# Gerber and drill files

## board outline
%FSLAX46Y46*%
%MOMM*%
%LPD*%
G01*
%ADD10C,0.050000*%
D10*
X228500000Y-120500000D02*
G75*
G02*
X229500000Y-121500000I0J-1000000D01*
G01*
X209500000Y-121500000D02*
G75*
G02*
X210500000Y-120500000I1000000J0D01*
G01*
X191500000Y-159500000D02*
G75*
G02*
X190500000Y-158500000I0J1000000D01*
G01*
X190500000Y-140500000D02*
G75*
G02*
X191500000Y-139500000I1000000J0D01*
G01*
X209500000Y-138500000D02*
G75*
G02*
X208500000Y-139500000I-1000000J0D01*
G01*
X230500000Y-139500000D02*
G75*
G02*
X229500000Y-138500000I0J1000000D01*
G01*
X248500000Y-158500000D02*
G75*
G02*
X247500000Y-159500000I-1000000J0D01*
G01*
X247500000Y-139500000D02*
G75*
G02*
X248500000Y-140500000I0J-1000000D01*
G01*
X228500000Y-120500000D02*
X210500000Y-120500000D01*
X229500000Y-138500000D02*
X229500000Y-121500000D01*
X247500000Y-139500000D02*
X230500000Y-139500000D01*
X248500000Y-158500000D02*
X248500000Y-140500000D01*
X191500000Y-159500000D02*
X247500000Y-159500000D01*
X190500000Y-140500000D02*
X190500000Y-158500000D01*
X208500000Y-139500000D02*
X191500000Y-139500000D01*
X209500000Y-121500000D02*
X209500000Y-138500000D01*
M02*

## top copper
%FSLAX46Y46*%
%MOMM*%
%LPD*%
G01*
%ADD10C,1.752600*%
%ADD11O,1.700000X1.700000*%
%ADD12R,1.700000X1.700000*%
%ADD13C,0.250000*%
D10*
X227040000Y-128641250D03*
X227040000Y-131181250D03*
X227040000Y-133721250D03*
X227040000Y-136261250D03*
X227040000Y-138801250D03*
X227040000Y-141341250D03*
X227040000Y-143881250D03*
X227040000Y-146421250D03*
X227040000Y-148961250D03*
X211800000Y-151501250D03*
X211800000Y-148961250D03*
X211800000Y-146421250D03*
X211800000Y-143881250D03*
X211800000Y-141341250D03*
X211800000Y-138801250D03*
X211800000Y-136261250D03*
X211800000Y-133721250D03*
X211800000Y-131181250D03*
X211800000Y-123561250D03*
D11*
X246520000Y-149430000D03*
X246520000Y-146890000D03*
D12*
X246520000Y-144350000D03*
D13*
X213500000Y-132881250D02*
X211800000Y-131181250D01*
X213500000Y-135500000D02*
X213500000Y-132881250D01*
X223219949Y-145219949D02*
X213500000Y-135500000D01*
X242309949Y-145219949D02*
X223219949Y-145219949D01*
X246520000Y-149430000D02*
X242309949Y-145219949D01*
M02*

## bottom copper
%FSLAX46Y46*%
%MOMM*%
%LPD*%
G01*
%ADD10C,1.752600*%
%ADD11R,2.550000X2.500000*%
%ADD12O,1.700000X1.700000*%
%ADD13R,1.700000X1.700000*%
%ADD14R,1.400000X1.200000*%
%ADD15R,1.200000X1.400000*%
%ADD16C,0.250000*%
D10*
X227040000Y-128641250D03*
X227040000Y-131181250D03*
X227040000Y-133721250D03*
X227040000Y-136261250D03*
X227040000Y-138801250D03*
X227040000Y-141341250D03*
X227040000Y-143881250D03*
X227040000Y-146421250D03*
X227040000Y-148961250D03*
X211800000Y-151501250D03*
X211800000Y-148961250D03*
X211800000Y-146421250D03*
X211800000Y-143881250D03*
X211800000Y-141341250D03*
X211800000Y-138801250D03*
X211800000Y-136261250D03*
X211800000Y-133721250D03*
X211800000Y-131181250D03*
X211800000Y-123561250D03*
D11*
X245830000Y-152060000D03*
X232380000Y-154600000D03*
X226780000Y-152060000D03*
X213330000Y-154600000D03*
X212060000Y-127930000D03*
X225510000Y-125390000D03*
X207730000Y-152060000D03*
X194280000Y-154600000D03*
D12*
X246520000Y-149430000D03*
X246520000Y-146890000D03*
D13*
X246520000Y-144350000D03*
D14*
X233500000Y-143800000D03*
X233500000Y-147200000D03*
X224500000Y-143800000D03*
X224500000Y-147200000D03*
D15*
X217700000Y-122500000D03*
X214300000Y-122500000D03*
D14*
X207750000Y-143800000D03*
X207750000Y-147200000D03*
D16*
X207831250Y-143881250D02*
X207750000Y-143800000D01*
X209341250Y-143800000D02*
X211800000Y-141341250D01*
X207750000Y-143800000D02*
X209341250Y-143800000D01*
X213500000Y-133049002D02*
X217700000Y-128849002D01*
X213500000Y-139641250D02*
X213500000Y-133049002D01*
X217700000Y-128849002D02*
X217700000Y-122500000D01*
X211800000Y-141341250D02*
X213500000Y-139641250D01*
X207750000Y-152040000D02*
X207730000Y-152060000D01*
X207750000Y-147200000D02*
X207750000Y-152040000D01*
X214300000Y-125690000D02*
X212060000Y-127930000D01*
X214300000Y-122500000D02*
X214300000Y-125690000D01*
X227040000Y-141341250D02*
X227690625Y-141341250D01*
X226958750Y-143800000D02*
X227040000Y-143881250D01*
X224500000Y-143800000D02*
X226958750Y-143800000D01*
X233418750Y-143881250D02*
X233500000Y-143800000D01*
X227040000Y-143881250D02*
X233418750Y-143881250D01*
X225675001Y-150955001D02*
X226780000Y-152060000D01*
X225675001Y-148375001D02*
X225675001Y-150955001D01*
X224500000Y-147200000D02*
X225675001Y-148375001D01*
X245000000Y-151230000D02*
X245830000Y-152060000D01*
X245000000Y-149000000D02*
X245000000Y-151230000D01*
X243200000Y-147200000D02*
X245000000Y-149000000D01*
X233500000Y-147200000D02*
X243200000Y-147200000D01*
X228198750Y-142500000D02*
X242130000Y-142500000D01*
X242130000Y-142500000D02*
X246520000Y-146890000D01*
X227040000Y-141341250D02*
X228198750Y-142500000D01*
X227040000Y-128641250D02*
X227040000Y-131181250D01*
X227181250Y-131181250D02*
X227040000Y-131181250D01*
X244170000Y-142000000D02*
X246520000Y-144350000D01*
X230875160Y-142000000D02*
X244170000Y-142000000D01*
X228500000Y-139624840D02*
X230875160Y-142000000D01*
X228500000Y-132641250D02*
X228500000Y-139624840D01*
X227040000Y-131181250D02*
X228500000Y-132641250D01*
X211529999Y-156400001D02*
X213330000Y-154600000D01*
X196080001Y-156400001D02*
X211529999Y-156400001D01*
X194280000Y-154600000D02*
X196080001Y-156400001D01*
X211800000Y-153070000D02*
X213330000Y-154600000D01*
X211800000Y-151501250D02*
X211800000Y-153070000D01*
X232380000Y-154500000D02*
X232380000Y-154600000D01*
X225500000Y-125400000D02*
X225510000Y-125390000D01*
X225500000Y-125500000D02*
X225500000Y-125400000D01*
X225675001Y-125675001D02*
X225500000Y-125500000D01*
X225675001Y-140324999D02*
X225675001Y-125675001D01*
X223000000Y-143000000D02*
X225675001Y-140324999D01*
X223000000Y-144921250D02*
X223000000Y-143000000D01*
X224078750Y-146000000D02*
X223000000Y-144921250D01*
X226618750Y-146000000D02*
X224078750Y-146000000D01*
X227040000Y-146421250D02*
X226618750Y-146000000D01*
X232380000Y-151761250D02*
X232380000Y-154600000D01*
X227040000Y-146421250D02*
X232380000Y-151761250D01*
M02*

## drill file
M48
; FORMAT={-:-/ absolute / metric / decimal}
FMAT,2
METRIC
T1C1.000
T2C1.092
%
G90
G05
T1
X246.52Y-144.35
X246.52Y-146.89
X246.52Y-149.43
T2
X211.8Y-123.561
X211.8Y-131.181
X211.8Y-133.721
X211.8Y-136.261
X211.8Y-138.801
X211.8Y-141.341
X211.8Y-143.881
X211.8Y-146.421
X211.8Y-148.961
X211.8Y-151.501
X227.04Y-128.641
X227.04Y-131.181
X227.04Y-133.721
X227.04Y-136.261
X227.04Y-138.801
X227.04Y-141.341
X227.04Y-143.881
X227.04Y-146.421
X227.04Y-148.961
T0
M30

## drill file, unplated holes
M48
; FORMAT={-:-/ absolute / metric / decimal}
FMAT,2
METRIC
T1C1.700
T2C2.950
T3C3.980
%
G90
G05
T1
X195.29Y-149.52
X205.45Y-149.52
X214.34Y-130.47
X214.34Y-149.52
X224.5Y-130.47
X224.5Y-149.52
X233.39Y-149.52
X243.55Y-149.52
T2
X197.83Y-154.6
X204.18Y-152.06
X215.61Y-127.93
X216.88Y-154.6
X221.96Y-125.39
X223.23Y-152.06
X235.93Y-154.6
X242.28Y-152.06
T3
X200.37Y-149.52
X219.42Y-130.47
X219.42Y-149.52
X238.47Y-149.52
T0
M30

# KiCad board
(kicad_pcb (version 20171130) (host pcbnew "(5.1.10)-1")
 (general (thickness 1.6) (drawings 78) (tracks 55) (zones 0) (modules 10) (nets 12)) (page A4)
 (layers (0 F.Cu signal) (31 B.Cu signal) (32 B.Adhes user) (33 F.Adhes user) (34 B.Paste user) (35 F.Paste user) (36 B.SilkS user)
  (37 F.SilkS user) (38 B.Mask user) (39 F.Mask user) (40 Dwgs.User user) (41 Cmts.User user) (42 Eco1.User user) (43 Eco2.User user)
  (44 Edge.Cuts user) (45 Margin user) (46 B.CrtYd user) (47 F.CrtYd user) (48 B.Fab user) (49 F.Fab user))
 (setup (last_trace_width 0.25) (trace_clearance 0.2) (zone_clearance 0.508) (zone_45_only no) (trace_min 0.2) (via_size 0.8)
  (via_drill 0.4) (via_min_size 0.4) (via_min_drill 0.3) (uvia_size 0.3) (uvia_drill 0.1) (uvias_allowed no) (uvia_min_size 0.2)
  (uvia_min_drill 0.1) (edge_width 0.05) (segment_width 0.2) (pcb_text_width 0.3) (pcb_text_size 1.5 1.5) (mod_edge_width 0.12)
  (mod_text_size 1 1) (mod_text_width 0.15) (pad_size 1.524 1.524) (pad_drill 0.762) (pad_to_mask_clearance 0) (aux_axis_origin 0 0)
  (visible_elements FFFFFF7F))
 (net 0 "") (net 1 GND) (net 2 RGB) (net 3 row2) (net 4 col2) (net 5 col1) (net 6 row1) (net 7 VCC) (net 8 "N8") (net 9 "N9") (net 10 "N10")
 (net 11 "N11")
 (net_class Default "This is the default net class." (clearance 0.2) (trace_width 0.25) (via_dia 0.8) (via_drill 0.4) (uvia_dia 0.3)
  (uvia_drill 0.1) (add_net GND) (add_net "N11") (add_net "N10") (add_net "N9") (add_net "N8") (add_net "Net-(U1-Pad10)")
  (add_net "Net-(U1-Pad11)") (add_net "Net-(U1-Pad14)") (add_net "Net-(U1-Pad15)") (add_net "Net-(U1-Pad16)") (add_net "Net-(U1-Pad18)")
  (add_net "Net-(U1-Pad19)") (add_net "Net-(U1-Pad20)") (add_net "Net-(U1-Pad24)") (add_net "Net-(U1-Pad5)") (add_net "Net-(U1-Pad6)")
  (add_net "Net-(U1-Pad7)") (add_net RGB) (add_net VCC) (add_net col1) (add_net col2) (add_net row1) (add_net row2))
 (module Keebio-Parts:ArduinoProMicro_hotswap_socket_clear (layer B.Cu) (at 219.42 137.53125 270)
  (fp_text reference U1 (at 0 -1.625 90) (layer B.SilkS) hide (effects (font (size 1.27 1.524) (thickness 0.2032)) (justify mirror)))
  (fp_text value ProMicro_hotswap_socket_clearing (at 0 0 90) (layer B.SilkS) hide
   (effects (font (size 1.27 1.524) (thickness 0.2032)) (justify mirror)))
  (pad 3 thru_hole circle (at -8.89 -7.62 270) (size 1.7526 1.7526) (drill 1.0922) (layers *.Cu *.SilkS *.Mask) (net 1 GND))
  (pad 4 thru_hole circle (at -6.35 -7.62 270) (size 1.7526 1.7526) (drill 1.0922) (layers *.Cu *.SilkS *.Mask) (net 1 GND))
  (pad 5 thru_hole circle (at -3.81 -7.62 270) (size 1.7526 1.7526) (drill 1.0922) (layers *.Cu *.SilkS *.Mask))
  (pad 6 thru_hole circle (at -1.27 -7.62 270) (size 1.7526 1.7526) (drill 1.0922) (layers *.Cu *.SilkS *.Mask))
  (pad 7 thru_hole circle (at 1.27 -7.62 270) (size 1.7526 1.7526) (drill 1.0922) (layers *.Cu *.SilkS *.Mask))
  (pad 8 thru_hole circle (at 3.81 -7.62 270) (size 1.7526 1.7526) (drill 1.0922) (layers *.Cu *.SilkS *.Mask) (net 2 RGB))
  (pad 9 thru_hole circle (at 6.35 -7.62 270) (size 1.7526 1.7526) (drill 1.0922) (layers *.Cu *.SilkS *.Mask) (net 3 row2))
  (pad 10 thru_hole circle (at 8.89 -7.62 270) (size 1.7526 1.7526) (drill 1.0922) (layers *.Cu *.SilkS *.Mask) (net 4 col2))
  (pad 11 thru_hole circle (at 11.43 -7.62 270) (size 1.7526 1.7526) (drill 1.0922) (layers *.Cu *.SilkS *.Mask))
  (pad 13 thru_hole circle (at 13.97 7.62 270) (size 1.7526 1.7526) (drill 1.0922) (layers *.Cu *.SilkS *.Mask) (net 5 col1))
  (pad 14 thru_hole circle (at 11.43 7.62 270) (size 1.7526 1.7526) (drill 1.0922) (layers *.Cu *.SilkS *.Mask))
  (pad 15 thru_hole circle (at 8.89 7.62 270) (size 1.7526 1.7526) (drill 1.0922) (layers *.Cu *.SilkS *.Mask))
  (pad 16 thru_hole circle (at 6.35 7.62 270) (size 1.7526 1.7526) (drill 1.0922) (layers *.Cu *.SilkS *.Mask))
  (pad 17 thru_hole circle (at 3.81 7.62 270) (size 1.7526 1.7526) (drill 1.0922) (layers *.Cu *.SilkS *.Mask) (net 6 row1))
  (pad 18 thru_hole circle (at 1.27 7.62 270) (size 1.7526 1.7526) (drill 1.0922) (layers *.Cu *.SilkS *.Mask))
  (pad 19 thru_hole circle (at -1.27 7.62 270) (size 1.7526 1.7526) (drill 1.0922) (layers *.Cu *.SilkS *.Mask))
  (pad 20 thru_hole circle (at -3.81 7.62 270) (size 1.7526 1.7526) (drill 1.0922) (layers *.Cu *.SilkS *.Mask))
  (pad 21 thru_hole circle (at -6.35 7.62 270) (size 1.7526 1.7526) (drill 1.0922) (layers *.Cu *.SilkS *.Mask) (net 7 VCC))
  (pad 24 thru_hole circle (at -13.97 7.62 270) (size 1.7526 1.7526) (drill 1.0922) (layers *.Cu *.SilkS *.Mask)))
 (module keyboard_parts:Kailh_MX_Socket (layer F.Cu) (at 238.47 149.52)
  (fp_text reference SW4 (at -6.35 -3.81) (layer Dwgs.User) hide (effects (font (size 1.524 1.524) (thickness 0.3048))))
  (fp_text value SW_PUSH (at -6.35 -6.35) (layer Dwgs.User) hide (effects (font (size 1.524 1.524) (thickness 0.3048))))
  (pad 1 smd rect (at 7.36 2.54) (size 2.55 2.5) (layers B.Cu B.Paste B.Mask) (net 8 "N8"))
  (pad "" np_thru_hole circle (at 0 0) (size 3.98018 3.98018) (drill 3.98018) (layers *.Cu *.Mask))
  (pad "" np_thru_hole circle (at -2.54 5.08) (size 2.95 2.95) (drill 2.95) (layers *.Cu *.Mask))
  (pad "" np_thru_hole circle (at 3.81 2.54) (size 2.95 2.95) (drill 2.95) (layers *.Cu *.Mask))
  (pad 2 smd rect (at -6.09 5.08) (size 2.55 2.5) (layers B.Cu B.Paste B.Mask) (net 4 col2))
  (pad "" np_thru_hole circle (at -5.08 0) (size 1.7 1.7) (drill 1.7) (layers *.Cu *.Mask))
  (pad "" np_thru_hole circle (at 5.08 0) (size 1.7 1.7) (drill 1.7) (layers *.Cu *.Mask)))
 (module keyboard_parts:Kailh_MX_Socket (layer F.Cu) (at 219.42 149.52)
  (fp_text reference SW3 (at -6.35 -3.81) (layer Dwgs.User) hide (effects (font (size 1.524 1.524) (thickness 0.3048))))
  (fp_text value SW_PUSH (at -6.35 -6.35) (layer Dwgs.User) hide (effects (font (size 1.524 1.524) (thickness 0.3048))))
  (pad 1 smd rect (at 7.36 2.54) (size 2.55 2.5) (layers B.Cu B.Paste B.Mask) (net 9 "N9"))
  (pad "" np_thru_hole circle (at 0 0) (size 3.98018 3.98018) (drill 3.98018) (layers *.Cu *.Mask))
  (pad "" np_thru_hole circle (at -2.54 5.08) (size 2.95 2.95) (drill 2.95) (layers *.Cu *.Mask))
  (pad "" np_thru_hole circle (at 3.81 2.54) (size 2.95 2.95) (drill 2.95) (layers *.Cu *.Mask))
  (pad 2 smd rect (at -6.09 5.08) (size 2.55 2.5) (layers B.Cu B.Paste B.Mask) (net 5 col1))
  (pad "" np_thru_hole circle (at -5.08 0) (size 1.7 1.7) (drill 1.7) (layers *.Cu *.Mask))
  (pad "" np_thru_hole circle (at 5.08 0) (size 1.7 1.7) (drill 1.7) (layers *.Cu *.Mask)))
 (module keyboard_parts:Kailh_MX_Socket (layer F.Cu) (at 219.42 130.47 180)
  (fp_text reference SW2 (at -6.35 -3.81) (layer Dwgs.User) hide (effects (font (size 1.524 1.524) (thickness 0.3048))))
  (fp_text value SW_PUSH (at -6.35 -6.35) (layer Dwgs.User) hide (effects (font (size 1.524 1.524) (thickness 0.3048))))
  (pad 1 smd rect (at 7.36 2.54 180) (size 2.55 2.5) (layers B.Cu B.Paste B.Mask) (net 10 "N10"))
  (pad "" np_thru_hole circle (at 0 0 180) (size 3.98018 3.98018) (drill 3.98018) (layers *.Cu *.Mask))
  (pad "" np_thru_hole circle (at -2.54 5.08 180) (size 2.95 2.95) (drill 2.95) (layers *.Cu *.Mask))
  (pad "" np_thru_hole circle (at 3.81 2.54 180) (size 2.95 2.95) (drill 2.95) (layers *.Cu *.Mask))
  (pad 2 smd rect (at -6.09 5.08 180) (size 2.55 2.5) (layers B.Cu B.Paste B.Mask) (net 4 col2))
  (pad "" np_thru_hole circle (at -5.08 0 180) (size 1.7 1.7) (drill 1.7) (layers *.Cu *.Mask))
  (pad "" np_thru_hole circle (at 5.08 0 180) (size 1.7 1.7) (drill 1.7) (layers *.Cu *.Mask)))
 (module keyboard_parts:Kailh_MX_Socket (layer F.Cu) (at 200.37 149.52)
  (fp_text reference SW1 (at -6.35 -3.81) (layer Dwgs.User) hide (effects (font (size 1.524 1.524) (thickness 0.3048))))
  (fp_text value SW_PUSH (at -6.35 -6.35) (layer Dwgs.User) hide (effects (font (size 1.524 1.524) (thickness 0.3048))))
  (pad 1 smd rect (at 7.36 2.54) (size 2.55 2.5) (layers B.Cu B.Paste B.Mask) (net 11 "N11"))
  (pad "" np_thru_hole circle (at 0 0) (size 3.98018 3.98018) (drill 3.98018) (layers *.Cu *.Mask))
  (pad "" np_thru_hole circle (at -2.54 5.08) (size 2.95 2.95) (drill 2.95) (layers *.Cu *.Mask))
  (pad "" np_thru_hole circle (at 3.81 2.54) (size 2.95 2.95) (drill 2.95) (layers *.Cu *.Mask))
  (pad 2 smd rect (at -6.09 5.08) (size 2.55 2.5) (layers B.Cu B.Paste B.Mask) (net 5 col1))
  (pad "" np_thru_hole circle (at -5.08 0) (size 1.7 1.7) (drill 1.7) (layers *.Cu *.Mask))
  (pad "" np_thru_hole circle (at 5.08 0) (size 1.7 1.7) (drill 1.7) (layers *.Cu *.Mask)))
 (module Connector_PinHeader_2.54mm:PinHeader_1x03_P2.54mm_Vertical (layer F.Cu) (at 246.52 144.35)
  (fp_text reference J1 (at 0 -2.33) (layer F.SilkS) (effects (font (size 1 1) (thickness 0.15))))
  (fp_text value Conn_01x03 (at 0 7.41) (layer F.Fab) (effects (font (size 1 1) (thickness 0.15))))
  (pad 3 thru_hole oval (at 0 5.08) (size 1.7 1.7) (drill 1) (layers *.Cu *.Mask) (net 7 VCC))
  (pad 2 thru_hole oval (at 0 2.54) (size 1.7 1.7) (drill 1) (layers *.Cu *.Mask) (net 2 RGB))
  (pad 1 thru_hole rect (at 0 0) (size 1.7 1.7) (drill 1) (layers *.Cu *.Mask) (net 1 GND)))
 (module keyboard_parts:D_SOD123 (layer B.Cu) (at 233.5 145.5 270)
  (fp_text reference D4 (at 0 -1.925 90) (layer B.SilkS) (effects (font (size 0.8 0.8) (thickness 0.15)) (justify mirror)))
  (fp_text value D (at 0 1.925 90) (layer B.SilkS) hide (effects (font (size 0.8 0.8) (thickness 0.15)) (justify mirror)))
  (pad 1 smd rect (at -1.7 0 270) (size 1.2 1.4) (layers B.Cu B.Paste B.Mask) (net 3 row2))
  (pad 2 smd rect (at 1.7 0 270) (size 1.2 1.4) (layers B.Cu B.Paste B.Mask) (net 8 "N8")))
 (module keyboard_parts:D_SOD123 (layer B.Cu) (at 224.5 145.5 270)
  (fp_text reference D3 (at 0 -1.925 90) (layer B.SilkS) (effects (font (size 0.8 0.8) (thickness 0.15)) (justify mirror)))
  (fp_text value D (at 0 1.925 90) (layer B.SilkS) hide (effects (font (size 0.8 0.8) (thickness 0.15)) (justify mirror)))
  (pad 1 smd rect (at -1.7 0 270) (size 1.2 1.4) (layers B.Cu B.Paste B.Mask) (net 3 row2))
  (pad 2 smd rect (at 1.7 0 270) (size 1.2 1.4) (layers B.Cu B.Paste B.Mask) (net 9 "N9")))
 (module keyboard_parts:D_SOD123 (layer B.Cu) (at 216 122.5 180)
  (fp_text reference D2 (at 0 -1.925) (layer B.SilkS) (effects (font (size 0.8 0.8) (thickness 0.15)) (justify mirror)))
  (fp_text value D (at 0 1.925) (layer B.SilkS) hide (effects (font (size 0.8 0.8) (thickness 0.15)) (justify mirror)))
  (pad 1 smd rect (at -1.7 0 180) (size 1.2 1.4) (layers B.Cu B.Paste B.Mask) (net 6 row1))
  (pad 2 smd rect (at 1.7 0 180) (size 1.2 1.4) (layers B.Cu B.Paste B.Mask) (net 10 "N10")))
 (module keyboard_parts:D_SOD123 (layer B.Cu) (at 207.75 145.5 270)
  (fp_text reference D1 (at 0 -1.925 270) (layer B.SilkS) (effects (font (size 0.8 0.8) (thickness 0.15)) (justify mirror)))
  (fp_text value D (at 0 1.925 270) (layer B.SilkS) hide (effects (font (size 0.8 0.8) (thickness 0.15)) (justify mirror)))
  (pad 1 smd rect (at -1.7 0 270) (size 1.2 1.4) (layers B.Cu B.Paste B.Mask) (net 6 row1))
  (pad 2 smd rect (at 1.7 0 270) (size 1.2 1.4) (layers B.Cu B.Paste B.Mask) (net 11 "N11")))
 (gr_arc (start 228.5 121.5) (end 229.5 121.5) (angle -90) (layer Edge.Cuts) (width 0.05))
 (gr_arc (start 210.5 121.5) (end 210.5 120.5) (angle -90) (layer Edge.Cuts) (width 0.05))
 (gr_arc (start 191.5 158.5) (end 190.5 158.5) (angle -90) (layer Edge.Cuts) (width 0.05))
 (gr_arc (start 191.5 140.5) (end 191.5 139.5) (angle -90) (layer Edge.Cuts) (width 0.05))
 (gr_arc (start 208.5 138.5) (end 208.5 139.5) (angle -90) (layer Edge.Cuts) (width 0.05))
 (gr_arc (start 230.5 138.5) (end 229.5 138.5) (angle -90) (layer Edge.Cuts) (width 0.05))
 (gr_arc (start 247.5 158.5) (end 247.5 159.5) (angle -90) (layer Edge.Cuts) (width 0.05))
 (gr_arc (start 247.5 140.5) (end 248.5 140.5) (angle -90) (layer Edge.Cuts) (width 0.05))
 (gr_line (start 228.5 120.5) (end 210.5 120.5) (layer Edge.Cuts) (width 0.05))
 (gr_line (start 229.5 138.5) (end 229.5 121.5) (layer Edge.Cuts) (width 0.05))
 (gr_line (start 247.5 139.5) (end 230.5 139.5) (layer Edge.Cuts) (width 0.05))
 (gr_line (start 248.5 158.5) (end 248.5 140.5) (layer Edge.Cuts) (width 0.05))
 (gr_line (start 191.5 159.5) (end 247.5 159.5) (layer Edge.Cuts) (width 0.05))
 (gr_line (start 190.5 140.5) (end 190.5 158.5) (layer Edge.Cuts) (width 0.05))
 (gr_line (start 208.5 139.5) (end 191.5 139.5) (layer Edge.Cuts) (width 0.05))
 (gr_line (start 209.5 121.5) (end 209.5 138.5) (layer Edge.Cuts) (width 0.05))
 (segment (start 207.83125 143.88125) (end 207.75 143.8) (width 0.25) (layer B.Cu) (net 6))
 (segment (start 209.34125 143.8) (end 211.8 141.34125) (width 0.25) (layer B.Cu) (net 6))
 (segment (start 207.75 143.8) (end 209.34125 143.8) (width 0.25) (layer B.Cu) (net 6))
 (segment (start 213.5 133.049002) (end 217.7 128.849002) (width 0.25) (layer B.Cu) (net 6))
 (segment (start 213.5 139.64125) (end 213.5 133.049002) (width 0.25) (layer B.Cu) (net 6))
 (segment (start 217.7 128.849002) (end 217.7 122.5) (width 0.25) (layer B.Cu) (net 6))
 (segment (start 211.8 141.34125) (end 213.5 139.64125) (width 0.25) (layer B.Cu) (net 6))
 (segment (start 207.75 152.04) (end 207.73 152.06) (width 0.25) (layer B.Cu) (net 11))
 (segment (start 207.75 147.2) (end 207.75 152.04) (width 0.25) (layer B.Cu) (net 11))
 (segment (start 214.3 125.69) (end 212.06 127.93) (width 0.25) (layer B.Cu) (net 10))
 (segment (start 214.3 122.5) (end 214.3 125.69) (width 0.25) (layer B.Cu) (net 10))
 (segment (start 227.04 141.34125) (end 227.690625 141.34125) (width 0.25) (layer B.Cu) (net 2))
 (segment (start 226.95875 143.8) (end 227.04 143.88125) (width 0.25) (layer B.Cu) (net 3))
 (segment (start 224.5 143.8) (end 226.95875 143.8) (width 0.25) (layer B.Cu) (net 3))
 (segment (start 233.41875 143.88125) (end 233.5 143.8) (width 0.25) (layer B.Cu) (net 3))
 (segment (start 227.04 143.88125) (end 233.41875 143.88125) (width 0.25) (layer B.Cu) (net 3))
 (segment (start 225.675001 150.955001) (end 226.78 152.06) (width 0.25) (layer B.Cu) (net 9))
 (segment (start 225.675001 148.375001) (end 225.675001 150.955001) (width 0.25) (layer B.Cu) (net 9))
 (segment (start 224.5 147.2) (end 225.675001 148.375001) (width 0.25) (layer B.Cu) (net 9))
 (segment (start 245 151.23) (end 245.83 152.06) (width 0.25) (layer B.Cu) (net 8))
 (segment (start 245 149) (end 245 151.23) (width 0.25) (layer B.Cu) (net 8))
 (segment (start 243.2 147.2) (end 245 149) (width 0.25) (layer B.Cu) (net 8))
 (segment (start 233.5 147.2) (end 243.2 147.2) (width 0.25) (layer B.Cu) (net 8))
 (segment (start 213.5 132.88125) (end 211.8 131.18125) (width 0.25) (layer F.Cu) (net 7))
 (segment (start 213.5 135.5) (end 213.5 132.88125) (width 0.25) (layer F.Cu) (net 7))
 (segment (start 223.219949 145.219949) (end 213.5 135.5) (width 0.25) (layer F.Cu) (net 7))
 (segment (start 242.309949 145.219949) (end 223.219949 145.219949) (width 0.25) (layer F.Cu) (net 7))
 (segment (start 246.52 149.43) (end 242.309949 145.219949) (width 0.25) (layer F.Cu) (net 7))
 (segment (start 228.19875 142.5) (end 242.13 142.5) (width 0.25) (layer B.Cu) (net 2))
 (segment (start 242.13 142.5) (end 246.52 146.89) (width 0.25) (layer B.Cu) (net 2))
 (segment (start 227.04 141.34125) (end 228.19875 142.5) (width 0.25) (layer B.Cu) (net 2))
 (segment (start 227.04 128.64125) (end 227.04 131.18125) (width 0.25) (layer B.Cu) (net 1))
 (segment (start 227.18125 131.18125) (end 227.04 131.18125) (width 0.25) (layer B.Cu) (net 1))
 (segment (start 244.17 142) (end 246.52 144.35) (width 0.25) (layer B.Cu) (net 1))
 (segment (start 230.87516 142) (end 244.17 142) (width 0.25) (layer B.Cu) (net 1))
 (segment (start 228.5 139.62484) (end 230.87516 142) (width 0.25) (layer B.Cu) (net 1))
 (segment (start 228.5 132.64125) (end 228.5 139.62484) (width 0.25) (layer B.Cu) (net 1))
 (segment (start 227.04 131.18125) (end 228.5 132.64125) (width 0.25) (layer B.Cu) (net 1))
 (segment (start 211.529999 156.400001) (end 213.33 154.6) (width 0.25) (layer B.Cu) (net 5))
 (segment (start 196.080001 156.400001) (end 211.529999 156.400001) (width 0.25) (layer B.Cu) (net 5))
 (segment (start 194.28 154.6) (end 196.080001 156.400001) (width 0.25) (layer B.Cu) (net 5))
 (segment (start 211.8 153.07) (end 213.33 154.6) (width 0.25) (layer B.Cu) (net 5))
 (segment (start 211.8 151.50125) (end 211.8 153.07) (width 0.25) (layer B.Cu) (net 5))
 (segment (start 232.38 154.5) (end 232.38 154.6) (width 0.25) (layer B.Cu) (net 4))
 (segment (start 225.5 125.4) (end 225.51 125.39) (width 0.25) (layer B.Cu) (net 4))
 (segment (start 225.5 125.5) (end 225.5 125.4) (width 0.25) (layer B.Cu) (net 4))
 (segment (start 225.675001 125.675001) (end 225.5 125.5) (width 0.25) (layer B.Cu) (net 4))
 (segment (start 225.675001 140.324999) (end 225.675001 125.675001) (width 0.25) (layer B.Cu) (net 4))
 (segment (start 223 143) (end 225.675001 140.324999) (width 0.25) (layer B.Cu) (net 4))
 (segment (start 223 144.92125) (end 223 143) (width 0.25) (layer B.Cu) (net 4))
 (segment (start 224.07875 146) (end 223 144.92125) (width 0.25) (layer B.Cu) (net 4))
 (segment (start 226.61875 146) (end 224.07875 146) (width 0.25) (layer B.Cu) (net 4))
 (segment (start 227.04 146.42125) (end 226.61875 146) (width 0.25) (layer B.Cu) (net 4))
 (segment (start 232.38 151.76125) (end 232.38 154.6) (width 0.25) (layer B.Cu) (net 4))
 (segment (start 227.04 146.42125) (end 232.38 151.76125) (width 0.25) (layer B.Cu) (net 4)))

